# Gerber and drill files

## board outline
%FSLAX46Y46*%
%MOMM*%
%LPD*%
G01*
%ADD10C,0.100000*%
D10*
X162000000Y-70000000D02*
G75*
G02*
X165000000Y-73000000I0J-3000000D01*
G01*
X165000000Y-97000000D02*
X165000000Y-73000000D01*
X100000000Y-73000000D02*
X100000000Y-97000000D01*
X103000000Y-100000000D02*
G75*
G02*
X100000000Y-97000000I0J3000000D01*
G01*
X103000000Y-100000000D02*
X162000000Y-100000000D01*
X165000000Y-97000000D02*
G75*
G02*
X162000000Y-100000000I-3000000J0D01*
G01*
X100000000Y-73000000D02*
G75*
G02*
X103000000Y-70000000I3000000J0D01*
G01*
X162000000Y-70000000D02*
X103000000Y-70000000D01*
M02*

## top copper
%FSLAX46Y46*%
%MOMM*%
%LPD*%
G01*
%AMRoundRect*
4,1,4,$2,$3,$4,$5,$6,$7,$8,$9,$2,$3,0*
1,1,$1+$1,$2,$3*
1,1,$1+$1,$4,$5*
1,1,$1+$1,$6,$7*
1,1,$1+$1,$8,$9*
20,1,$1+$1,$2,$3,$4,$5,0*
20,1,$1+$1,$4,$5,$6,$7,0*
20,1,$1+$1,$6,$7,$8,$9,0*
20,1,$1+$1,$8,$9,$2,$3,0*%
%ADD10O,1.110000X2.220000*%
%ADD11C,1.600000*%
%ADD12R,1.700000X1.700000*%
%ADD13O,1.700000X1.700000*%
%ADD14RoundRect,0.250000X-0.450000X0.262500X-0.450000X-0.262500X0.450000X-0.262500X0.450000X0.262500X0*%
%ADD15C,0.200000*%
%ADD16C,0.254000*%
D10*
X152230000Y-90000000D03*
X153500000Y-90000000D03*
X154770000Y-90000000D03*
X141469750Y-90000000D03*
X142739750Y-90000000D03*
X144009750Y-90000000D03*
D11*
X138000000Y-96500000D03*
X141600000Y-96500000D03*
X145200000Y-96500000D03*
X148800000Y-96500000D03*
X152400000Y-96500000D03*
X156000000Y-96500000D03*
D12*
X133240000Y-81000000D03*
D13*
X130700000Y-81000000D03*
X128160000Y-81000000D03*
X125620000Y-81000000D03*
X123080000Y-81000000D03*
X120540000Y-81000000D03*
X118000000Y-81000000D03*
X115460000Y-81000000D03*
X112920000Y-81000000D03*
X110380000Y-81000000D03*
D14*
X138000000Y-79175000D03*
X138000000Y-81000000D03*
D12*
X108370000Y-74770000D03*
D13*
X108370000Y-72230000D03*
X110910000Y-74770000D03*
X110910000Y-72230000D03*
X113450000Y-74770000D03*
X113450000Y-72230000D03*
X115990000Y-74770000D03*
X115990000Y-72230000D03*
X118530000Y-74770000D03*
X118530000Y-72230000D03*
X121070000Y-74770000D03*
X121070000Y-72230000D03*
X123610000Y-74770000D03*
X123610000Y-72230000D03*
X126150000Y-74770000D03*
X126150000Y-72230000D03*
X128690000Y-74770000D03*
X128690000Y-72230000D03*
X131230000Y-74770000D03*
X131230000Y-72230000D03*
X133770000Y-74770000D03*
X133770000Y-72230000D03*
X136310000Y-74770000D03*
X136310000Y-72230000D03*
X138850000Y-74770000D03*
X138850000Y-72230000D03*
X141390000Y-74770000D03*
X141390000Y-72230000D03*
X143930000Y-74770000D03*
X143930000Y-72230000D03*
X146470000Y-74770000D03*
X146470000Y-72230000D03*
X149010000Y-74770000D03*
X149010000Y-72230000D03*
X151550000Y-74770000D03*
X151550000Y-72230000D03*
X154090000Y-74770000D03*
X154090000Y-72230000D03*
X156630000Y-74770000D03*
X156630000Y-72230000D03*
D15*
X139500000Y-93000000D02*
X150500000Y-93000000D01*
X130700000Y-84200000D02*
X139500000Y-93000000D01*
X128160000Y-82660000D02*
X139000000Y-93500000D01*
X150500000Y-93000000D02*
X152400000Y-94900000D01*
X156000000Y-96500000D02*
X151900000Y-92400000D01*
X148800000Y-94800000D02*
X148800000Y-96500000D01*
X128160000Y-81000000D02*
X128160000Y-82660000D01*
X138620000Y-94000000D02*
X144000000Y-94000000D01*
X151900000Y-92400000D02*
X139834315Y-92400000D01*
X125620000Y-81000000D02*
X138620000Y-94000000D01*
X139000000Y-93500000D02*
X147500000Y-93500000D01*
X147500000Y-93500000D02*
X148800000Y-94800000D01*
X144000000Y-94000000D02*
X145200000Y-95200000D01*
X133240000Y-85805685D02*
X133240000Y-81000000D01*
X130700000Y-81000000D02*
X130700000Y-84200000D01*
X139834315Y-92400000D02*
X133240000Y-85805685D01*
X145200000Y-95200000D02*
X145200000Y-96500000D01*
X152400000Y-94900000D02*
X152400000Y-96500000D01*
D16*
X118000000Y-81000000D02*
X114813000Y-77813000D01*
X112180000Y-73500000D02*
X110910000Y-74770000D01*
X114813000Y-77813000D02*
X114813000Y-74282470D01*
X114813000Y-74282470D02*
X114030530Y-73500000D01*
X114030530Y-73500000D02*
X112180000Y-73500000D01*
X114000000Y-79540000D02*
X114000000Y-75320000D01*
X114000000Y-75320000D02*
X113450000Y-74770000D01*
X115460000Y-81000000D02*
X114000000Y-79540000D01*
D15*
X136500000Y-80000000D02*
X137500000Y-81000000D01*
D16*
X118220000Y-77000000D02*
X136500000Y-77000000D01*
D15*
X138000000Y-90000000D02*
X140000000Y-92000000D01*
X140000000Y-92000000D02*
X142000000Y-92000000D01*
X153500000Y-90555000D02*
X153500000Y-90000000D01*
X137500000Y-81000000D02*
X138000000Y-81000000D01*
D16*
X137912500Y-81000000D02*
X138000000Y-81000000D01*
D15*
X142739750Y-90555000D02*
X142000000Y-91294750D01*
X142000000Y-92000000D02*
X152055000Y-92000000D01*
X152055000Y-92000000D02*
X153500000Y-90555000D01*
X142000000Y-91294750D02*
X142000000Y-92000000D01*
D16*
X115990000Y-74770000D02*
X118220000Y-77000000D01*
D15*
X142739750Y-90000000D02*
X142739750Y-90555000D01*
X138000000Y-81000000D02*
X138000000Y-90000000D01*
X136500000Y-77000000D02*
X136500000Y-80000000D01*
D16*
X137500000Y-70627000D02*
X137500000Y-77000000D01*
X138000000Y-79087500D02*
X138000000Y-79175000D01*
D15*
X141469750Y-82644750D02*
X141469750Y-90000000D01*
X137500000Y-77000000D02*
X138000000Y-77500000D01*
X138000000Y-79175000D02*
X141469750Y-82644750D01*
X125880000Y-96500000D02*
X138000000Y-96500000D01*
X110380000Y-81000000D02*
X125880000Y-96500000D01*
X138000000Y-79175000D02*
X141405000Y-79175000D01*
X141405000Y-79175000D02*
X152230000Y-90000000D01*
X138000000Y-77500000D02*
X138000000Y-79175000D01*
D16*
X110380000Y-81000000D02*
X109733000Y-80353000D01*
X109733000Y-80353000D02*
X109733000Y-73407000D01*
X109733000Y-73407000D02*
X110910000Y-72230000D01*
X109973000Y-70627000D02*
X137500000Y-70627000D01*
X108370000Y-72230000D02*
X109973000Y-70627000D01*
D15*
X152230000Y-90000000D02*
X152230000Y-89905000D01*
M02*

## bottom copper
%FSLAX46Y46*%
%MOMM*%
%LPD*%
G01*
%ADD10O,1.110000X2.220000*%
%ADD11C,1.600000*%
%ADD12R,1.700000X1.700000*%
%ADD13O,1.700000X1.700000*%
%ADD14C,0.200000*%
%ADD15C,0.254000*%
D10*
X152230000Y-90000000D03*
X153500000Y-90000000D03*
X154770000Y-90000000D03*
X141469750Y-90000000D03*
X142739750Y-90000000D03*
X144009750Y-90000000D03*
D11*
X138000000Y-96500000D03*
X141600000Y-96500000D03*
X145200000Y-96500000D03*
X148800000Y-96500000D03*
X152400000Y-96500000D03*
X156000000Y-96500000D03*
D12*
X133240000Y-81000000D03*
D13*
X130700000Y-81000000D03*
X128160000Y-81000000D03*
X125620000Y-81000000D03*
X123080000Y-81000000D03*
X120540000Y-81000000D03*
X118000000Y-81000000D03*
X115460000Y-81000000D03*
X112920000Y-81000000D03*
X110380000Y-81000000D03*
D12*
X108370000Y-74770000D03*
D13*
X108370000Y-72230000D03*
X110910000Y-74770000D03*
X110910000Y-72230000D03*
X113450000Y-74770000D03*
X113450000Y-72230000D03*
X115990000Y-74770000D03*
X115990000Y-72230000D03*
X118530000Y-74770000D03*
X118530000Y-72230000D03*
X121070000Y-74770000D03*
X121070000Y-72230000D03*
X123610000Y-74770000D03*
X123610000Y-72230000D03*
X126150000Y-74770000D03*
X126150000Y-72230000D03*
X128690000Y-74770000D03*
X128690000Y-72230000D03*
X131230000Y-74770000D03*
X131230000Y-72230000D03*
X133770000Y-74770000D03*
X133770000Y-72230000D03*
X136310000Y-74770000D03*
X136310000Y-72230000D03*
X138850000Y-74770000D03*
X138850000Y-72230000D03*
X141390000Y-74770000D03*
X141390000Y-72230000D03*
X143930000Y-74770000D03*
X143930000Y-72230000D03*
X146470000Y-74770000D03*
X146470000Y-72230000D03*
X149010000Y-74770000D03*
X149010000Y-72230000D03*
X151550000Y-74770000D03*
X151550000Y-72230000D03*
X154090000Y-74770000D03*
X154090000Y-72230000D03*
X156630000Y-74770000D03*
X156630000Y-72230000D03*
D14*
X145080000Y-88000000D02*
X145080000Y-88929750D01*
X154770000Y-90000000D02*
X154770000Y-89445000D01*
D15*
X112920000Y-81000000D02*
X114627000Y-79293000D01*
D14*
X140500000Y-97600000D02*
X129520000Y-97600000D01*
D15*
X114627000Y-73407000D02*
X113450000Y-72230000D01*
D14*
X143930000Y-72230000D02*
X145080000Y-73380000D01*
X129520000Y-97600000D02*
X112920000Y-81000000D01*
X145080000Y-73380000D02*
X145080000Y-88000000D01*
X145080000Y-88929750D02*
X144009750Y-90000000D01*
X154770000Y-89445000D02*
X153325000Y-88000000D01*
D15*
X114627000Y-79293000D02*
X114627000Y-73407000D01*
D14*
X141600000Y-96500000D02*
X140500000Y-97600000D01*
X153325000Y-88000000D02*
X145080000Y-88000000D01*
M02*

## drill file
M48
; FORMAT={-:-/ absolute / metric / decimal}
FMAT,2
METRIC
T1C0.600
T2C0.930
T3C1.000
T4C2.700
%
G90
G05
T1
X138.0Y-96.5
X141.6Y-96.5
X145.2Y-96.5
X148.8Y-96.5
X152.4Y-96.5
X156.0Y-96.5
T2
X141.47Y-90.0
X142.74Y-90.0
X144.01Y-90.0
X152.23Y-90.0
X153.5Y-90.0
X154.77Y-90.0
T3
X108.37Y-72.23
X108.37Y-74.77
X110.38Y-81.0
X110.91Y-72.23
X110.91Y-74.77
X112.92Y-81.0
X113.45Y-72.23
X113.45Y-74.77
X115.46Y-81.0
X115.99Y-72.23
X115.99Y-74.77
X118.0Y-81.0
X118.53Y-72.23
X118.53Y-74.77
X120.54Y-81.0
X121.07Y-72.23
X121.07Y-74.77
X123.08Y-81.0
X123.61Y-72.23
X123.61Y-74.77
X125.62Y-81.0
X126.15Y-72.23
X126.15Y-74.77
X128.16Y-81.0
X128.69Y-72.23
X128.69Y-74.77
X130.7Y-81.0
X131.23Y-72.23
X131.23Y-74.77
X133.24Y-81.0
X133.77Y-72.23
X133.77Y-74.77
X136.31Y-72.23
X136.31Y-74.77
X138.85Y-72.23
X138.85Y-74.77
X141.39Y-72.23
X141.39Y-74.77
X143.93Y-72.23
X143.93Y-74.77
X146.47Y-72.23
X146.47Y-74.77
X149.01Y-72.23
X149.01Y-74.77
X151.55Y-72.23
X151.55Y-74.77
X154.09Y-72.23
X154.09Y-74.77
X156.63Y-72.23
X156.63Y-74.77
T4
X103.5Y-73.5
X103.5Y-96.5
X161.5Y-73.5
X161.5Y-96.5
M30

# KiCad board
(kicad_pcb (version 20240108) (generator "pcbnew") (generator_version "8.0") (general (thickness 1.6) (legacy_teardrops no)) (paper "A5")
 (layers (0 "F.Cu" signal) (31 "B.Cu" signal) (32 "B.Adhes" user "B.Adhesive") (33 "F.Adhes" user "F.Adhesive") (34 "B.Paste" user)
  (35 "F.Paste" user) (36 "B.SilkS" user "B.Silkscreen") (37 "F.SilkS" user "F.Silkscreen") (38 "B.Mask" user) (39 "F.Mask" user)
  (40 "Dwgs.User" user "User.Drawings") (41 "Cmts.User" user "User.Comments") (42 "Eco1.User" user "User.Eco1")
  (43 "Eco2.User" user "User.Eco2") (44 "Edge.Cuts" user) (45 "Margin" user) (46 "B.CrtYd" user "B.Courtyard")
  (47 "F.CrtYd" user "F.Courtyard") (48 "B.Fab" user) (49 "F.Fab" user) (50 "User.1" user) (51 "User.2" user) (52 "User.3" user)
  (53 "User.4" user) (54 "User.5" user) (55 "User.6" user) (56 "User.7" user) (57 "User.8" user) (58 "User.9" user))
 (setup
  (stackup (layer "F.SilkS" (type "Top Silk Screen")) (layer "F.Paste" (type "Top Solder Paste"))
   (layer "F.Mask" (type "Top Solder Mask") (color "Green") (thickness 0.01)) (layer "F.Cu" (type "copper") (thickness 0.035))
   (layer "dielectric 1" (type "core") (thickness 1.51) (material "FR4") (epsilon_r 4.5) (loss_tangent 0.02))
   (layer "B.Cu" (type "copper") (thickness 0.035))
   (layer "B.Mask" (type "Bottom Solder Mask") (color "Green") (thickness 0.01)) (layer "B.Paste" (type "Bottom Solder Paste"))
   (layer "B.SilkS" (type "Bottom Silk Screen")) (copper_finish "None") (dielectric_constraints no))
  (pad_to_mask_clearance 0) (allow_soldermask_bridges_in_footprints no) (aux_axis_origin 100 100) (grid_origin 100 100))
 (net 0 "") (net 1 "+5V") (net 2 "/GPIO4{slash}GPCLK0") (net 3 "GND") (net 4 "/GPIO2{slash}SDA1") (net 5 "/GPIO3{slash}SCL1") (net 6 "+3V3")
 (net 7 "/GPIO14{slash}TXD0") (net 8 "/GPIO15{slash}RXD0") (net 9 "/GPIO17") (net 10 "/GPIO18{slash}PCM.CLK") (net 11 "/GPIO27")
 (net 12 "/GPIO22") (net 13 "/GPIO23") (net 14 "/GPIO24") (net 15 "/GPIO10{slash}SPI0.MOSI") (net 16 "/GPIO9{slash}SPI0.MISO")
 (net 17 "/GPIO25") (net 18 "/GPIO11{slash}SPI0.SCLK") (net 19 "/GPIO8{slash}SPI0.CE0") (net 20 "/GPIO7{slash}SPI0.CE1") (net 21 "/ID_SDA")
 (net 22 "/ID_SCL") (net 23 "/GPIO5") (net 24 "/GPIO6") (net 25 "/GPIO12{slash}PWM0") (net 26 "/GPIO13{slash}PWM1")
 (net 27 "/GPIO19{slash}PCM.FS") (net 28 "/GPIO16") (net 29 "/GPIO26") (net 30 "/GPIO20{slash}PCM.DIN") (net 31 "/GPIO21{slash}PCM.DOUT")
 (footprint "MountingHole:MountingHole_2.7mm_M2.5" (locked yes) (layer "F.Cu") (at 161.5 73.5)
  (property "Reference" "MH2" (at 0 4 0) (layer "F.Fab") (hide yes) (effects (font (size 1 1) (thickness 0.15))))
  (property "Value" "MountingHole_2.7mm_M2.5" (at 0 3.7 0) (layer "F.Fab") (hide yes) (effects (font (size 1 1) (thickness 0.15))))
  (pad "" np_thru_hole circle (at 0 0) (size 2.7 2.7) (drill 2.7) (layers "*.Cu" "*.Mask")))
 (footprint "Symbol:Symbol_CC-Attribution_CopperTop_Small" (layer "F.Cu") (at 155.5 79)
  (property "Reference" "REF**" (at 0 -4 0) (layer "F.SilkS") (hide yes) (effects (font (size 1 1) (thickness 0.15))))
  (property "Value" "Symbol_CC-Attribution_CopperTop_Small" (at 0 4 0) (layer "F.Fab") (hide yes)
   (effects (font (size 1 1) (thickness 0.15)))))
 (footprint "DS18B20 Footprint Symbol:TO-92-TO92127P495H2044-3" (layer "F.Cu") (at 153.5 89.23975)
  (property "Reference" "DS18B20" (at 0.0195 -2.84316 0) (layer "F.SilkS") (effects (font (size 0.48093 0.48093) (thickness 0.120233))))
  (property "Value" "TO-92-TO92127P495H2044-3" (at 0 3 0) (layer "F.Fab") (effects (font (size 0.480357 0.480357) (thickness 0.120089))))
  (pad "1" thru_hole oval (at -1.27 0.76025) (size 1.11 2.22) (drill 0.93) (layers "*.Cu" "*.Mask") (remove_unused_layers no) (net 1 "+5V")
   (solder_mask_margin 0.102))
  (pad "2" thru_hole oval (at 0 0.76025) (size 1.11 2.22) (drill 0.93) (layers "*.Cu" "*.Mask") (remove_unused_layers no)
   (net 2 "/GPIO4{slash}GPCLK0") (solder_mask_margin 0.102))
  (pad "3" thru_hole oval (at 1.27 0.76025) (size 1.11 2.22) (drill 0.93) (layers "*.Cu" "*.Mask") (remove_unused_layers no) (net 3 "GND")
   (solder_mask_margin 0.102)))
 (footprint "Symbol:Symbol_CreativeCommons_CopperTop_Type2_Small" (layer "F.Cu") (at 149.5 79)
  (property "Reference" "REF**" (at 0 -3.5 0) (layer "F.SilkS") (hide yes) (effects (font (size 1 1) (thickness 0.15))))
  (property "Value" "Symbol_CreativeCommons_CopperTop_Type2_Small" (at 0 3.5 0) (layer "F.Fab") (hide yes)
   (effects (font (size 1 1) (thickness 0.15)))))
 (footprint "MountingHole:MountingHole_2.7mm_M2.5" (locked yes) (layer "F.Cu") (at 103.5 96.5)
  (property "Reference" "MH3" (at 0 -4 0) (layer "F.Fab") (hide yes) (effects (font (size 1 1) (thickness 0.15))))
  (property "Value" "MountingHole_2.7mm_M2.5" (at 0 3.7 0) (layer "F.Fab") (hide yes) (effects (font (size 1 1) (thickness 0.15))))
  (pad "" np_thru_hole circle (at 0 0) (size 2.7 2.7) (drill 2.7) (layers "*.Cu" "*.Mask")))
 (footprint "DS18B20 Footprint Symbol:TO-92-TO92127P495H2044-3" (layer "F.Cu") (at 142.73975 89.23975)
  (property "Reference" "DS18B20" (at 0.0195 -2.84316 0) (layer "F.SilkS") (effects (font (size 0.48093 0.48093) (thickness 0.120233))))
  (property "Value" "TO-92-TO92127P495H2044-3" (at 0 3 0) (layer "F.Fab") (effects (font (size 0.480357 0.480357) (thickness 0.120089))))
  (pad "1" thru_hole oval (at -1.27 0.76025) (size 1.11 2.22) (drill 0.93) (layers "*.Cu" "*.Mask") (remove_unused_layers no) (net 1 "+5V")
   (solder_mask_margin 0.102))
  (pad "2" thru_hole oval (at 0 0.76025) (size 1.11 2.22) (drill 0.93) (layers "*.Cu" "*.Mask") (remove_unused_layers no)
   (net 2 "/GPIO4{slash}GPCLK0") (solder_mask_margin 0.102))
  (pad "3" thru_hole oval (at 1.27 0.76025) (size 1.11 2.22) (drill 0.93) (layers "*.Cu" "*.Mask") (remove_unused_layers no) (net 3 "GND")
   (solder_mask_margin 0.102)))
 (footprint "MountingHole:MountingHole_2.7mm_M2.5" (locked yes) (layer "F.Cu") (at 103.5 73.5)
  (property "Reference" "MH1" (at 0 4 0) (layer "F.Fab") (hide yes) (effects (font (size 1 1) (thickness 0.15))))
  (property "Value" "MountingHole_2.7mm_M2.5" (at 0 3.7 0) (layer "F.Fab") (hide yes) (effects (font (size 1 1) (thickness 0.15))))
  (pad "" np_thru_hole circle (at 0 0) (size 2.7 2.7) (drill 2.7) (layers "*.Cu" "*.Mask")))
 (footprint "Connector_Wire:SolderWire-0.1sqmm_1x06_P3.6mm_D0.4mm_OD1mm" (layer "F.Cu") (at 138 96.5)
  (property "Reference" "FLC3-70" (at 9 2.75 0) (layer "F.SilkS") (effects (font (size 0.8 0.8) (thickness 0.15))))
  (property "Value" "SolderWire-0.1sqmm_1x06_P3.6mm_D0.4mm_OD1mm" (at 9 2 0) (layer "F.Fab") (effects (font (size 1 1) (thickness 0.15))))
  (pad "1" thru_hole circle (at 0 0) (size 1.6 1.6) (drill 0.6) (layers "*.Cu" "*.Mask") (remove_unused_layers no) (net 1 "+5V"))
  (pad "2" thru_hole circle (at 3.6 0) (size 1.6 1.6) (drill 0.6) (layers "*.Cu" "*.Mask") (remove_unused_layers no) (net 3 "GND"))
  (pad "3" thru_hole circle (at 7.2 0) (size 1.6 1.6) (drill 0.6) (layers "*.Cu" "*.Mask") (remove_unused_layers no))
  (pad "4" thru_hole circle (at 10.8 0) (size 1.6 1.6) (drill 0.6) (layers "*.Cu" "*.Mask") (remove_unused_layers no))
  (pad "5" thru_hole circle (at 14.4 0) (size 1.6 1.6) (drill 0.6) (layers "*.Cu" "*.Mask") (remove_unused_layers no))
  (pad "6" thru_hole circle (at 18 0) (size 1.6 1.6) (drill 0.6) (layers "*.Cu" "*.Mask") (remove_unused_layers no)))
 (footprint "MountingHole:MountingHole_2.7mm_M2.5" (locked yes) (layer "F.Cu") (at 161.5 96.5)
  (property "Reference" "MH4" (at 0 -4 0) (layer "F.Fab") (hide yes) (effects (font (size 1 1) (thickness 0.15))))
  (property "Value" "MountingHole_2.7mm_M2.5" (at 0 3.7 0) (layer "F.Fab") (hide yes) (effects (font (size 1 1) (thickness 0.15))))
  (pad "" np_thru_hole circle (at 0 0) (size 2.7 2.7) (drill 2.7) (layers "*.Cu" "*.Mask")))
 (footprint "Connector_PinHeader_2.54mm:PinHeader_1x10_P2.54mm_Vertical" (layer "F.Cu") (at 133.24 81 -90)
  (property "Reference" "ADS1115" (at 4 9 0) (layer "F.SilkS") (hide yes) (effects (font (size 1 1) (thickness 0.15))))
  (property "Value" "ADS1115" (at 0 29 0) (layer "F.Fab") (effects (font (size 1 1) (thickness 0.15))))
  (pad "1" thru_hole rect (at 0 0 270) (size 1.7 1.7) (drill 1) (layers "*.Cu" "*.Mask") (remove_unused_layers no))
  (pad "2" thru_hole oval (at 0 2.54 270) (size 1.7 1.7) (drill 1) (layers "*.Cu" "*.Mask") (remove_unused_layers no))
  (pad "3" thru_hole oval (at 0 5.08 270) (size 1.7 1.7) (drill 1) (layers "*.Cu" "*.Mask") (remove_unused_layers no))
  (pad "4" thru_hole oval (at 0 7.62 270) (size 1.7 1.7) (drill 1) (layers "*.Cu" "*.Mask") (remove_unused_layers no))
  (pad "5" thru_hole oval (at 0 10.16 270) (size 1.7 1.7) (drill 1) (layers "*.Cu" "*.Mask") (remove_unused_layers no))
  (pad "6" thru_hole oval (at 0 12.7 270) (size 1.7 1.7) (drill 1) (layers "*.Cu" "*.Mask") (remove_unused_layers no))
  (pad "7" thru_hole oval (at 0 15.24 270) (size 1.7 1.7) (drill 1) (layers "*.Cu" "*.Mask") (remove_unused_layers no)
   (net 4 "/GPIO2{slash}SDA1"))
  (pad "8" thru_hole oval (at 0 17.78 270) (size 1.7 1.7) (drill 1) (layers "*.Cu" "*.Mask") (remove_unused_layers no)
   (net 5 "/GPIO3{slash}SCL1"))
  (pad "9" thru_hole oval (at 0 20.32 270) (size 1.7 1.7) (drill 1) (layers "*.Cu" "*.Mask") (remove_unused_layers no) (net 3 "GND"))
  (pad "10" thru_hole oval (at 0 22.86 270) (size 1.7 1.7) (drill 1) (layers "*.Cu" "*.Mask") (remove_unused_layers no) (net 1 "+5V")))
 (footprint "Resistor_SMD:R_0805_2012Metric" (layer "F.Cu") (at 138 80.0875 -90)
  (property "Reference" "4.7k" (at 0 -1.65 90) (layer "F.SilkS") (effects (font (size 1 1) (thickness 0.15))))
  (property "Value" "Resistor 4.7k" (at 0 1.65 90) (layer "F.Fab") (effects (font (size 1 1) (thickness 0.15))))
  (pad "1" smd roundrect (at -0.9125 0 270) (size 1.025 1.4) (layers "F.Cu" "F.Paste" "F.Mask") (roundrect_rratio 0.243902) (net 1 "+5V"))
  (pad "2" smd roundrect (at 0.9125 0 270) (size 1.025 1.4) (layers "F.Cu" "F.Paste" "F.Mask") (roundrect_rratio 0.243902)
   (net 2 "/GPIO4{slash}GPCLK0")))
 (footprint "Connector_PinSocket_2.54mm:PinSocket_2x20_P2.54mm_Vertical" (layer "B.Cu") (at 108.37 74.77 -90)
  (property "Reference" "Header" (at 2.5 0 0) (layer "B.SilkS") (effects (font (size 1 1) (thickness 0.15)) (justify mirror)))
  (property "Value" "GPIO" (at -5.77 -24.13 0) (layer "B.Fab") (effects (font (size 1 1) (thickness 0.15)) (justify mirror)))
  (pad "1" thru_hole rect (at 0 0 270) (size 1.7 1.7) (drill 1) (layers "*.Cu" "*.Mask") (remove_unused_layers no) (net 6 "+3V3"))
  (pad "2" thru_hole oval (at -2.54 0 270) (size 1.7 1.7) (drill 1) (layers "*.Cu" "*.Mask") (remove_unused_layers no) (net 1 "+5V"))
  (pad "3" thru_hole oval (at 0 -2.54 270) (size 1.7 1.7) (drill 1) (layers "*.Cu" "*.Mask") (remove_unused_layers no)
   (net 4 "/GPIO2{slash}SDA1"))
  (pad "4" thru_hole oval (at -2.54 -2.54 270) (size 1.7 1.7) (drill 1) (layers "*.Cu" "*.Mask") (remove_unused_layers no) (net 1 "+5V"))
  (pad "5" thru_hole oval (at 0 -5.08 270) (size 1.7 1.7) (drill 1) (layers "*.Cu" "*.Mask") (remove_unused_layers no)
   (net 5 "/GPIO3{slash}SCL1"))
  (pad "6" thru_hole oval (at -2.54 -5.08 270) (size 1.7 1.7) (drill 1) (layers "*.Cu" "*.Mask") (remove_unused_layers no) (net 3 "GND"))
  (pad "7" thru_hole oval (at 0 -7.62 270) (size 1.7 1.7) (drill 1) (layers "*.Cu" "*.Mask") (remove_unused_layers no)
   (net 2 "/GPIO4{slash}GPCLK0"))
  (pad "8" thru_hole oval (at -2.54 -7.62 270) (size 1.7 1.7) (drill 1) (layers "*.Cu" "*.Mask") (remove_unused_layers no)
   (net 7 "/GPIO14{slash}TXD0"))
  (pad "9" thru_hole oval (at 0 -10.16 270) (size 1.7 1.7) (drill 1) (layers "*.Cu" "*.Mask") (remove_unused_layers no) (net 3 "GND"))
  (pad "10" thru_hole oval (at -2.54 -10.16 270) (size 1.7 1.7) (drill 1) (layers "*.Cu" "*.Mask") (remove_unused_layers no)
   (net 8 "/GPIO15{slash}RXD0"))
  (pad "11" thru_hole oval (at 0 -12.7 270) (size 1.7 1.7) (drill 1) (layers "*.Cu" "*.Mask") (remove_unused_layers no) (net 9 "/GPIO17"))
  (pad "12" thru_hole oval (at -2.54 -12.7 270) (size 1.7 1.7) (drill 1) (layers "*.Cu" "*.Mask") (remove_unused_layers no)
   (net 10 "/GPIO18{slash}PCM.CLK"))
  (pad "13" thru_hole oval (at 0 -15.24 270) (size 1.7 1.7) (drill 1) (layers "*.Cu" "*.Mask") (remove_unused_layers no) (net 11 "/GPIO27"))
  (pad "14" thru_hole oval (at -2.54 -15.24 270) (size 1.7 1.7) (drill 1) (layers "*.Cu" "*.Mask") (remove_unused_layers no) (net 3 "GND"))
  (pad "15" thru_hole oval (at 0 -17.78 270) (size 1.7 1.7) (drill 1) (layers "*.Cu" "*.Mask") (remove_unused_layers no) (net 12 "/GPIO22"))
  (pad "16" thru_hole oval (at -2.54 -17.78 270) (size 1.7 1.7) (drill 1) (layers "*.Cu" "*.Mask") (remove_unused_layers no)
   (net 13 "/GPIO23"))
  (pad "17" thru_hole oval (at 0 -20.32 270) (size 1.7 1.7) (drill 1) (layers "*.Cu" "*.Mask") (remove_unused_layers no) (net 6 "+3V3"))
  (pad "18" thru_hole oval (at -2.54 -20.32 270) (size 1.7 1.7) (drill 1) (layers "*.Cu" "*.Mask") (remove_unused_layers no)
   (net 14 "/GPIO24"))
  (pad "19" thru_hole oval (at 0 -22.86 270) (size 1.7 1.7) (drill 1) (layers "*.Cu" "*.Mask") (remove_unused_layers no)
   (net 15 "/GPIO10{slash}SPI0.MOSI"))
  (pad "20" thru_hole oval (at -2.54 -22.86 270) (size 1.7 1.7) (drill 1) (layers "*.Cu" "*.Mask") (remove_unused_layers no) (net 3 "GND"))
  (pad "21" thru_hole oval (at 0 -25.4 270) (size 1.7 1.7) (drill 1) (layers "*.Cu" "*.Mask") (remove_unused_layers no)
   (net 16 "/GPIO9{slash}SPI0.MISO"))
  (pad "22" thru_hole oval (at -2.54 -25.4 270) (size 1.7 1.7) (drill 1) (layers "*.Cu" "*.Mask") (remove_unused_layers no)
   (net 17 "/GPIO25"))
  (pad "23" thru_hole oval (at 0 -27.94 270) (size 1.7 1.7) (drill 1) (layers "*.Cu" "*.Mask") (remove_unused_layers no)
   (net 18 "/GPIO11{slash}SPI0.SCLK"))
  (pad "24" thru_hole oval (at -2.54 -27.94 270) (size 1.7 1.7) (drill 1) (layers "*.Cu" "*.Mask") (remove_unused_layers no)
   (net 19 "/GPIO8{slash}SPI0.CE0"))
  (pad "25" thru_hole oval (at 0 -30.48 270) (size 1.7 1.7) (drill 1) (layers "*.Cu" "*.Mask") (remove_unused_layers no) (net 3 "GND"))
  (pad "26" thru_hole oval (at -2.54 -30.48 270) (size 1.7 1.7) (drill 1) (layers "*.Cu" "*.Mask") (remove_unused_layers no)
   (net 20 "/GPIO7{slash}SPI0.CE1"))
  (pad "27" thru_hole oval (at 0 -33.02 270) (size 1.7 1.7) (drill 1) (layers "*.Cu" "*.Mask") (remove_unused_layers no) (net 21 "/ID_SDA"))
  (pad "28" thru_hole oval (at -2.54 -33.02 270) (size 1.7 1.7) (drill 1) (layers "*.Cu" "*.Mask") (remove_unused_layers no)
   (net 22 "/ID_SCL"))
  (pad "29" thru_hole oval (at 0 -35.56 270) (size 1.7 1.7) (drill 1) (layers "*.Cu" "*.Mask") (remove_unused_layers no) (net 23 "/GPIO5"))
  (pad "30" thru_hole oval (at -2.54 -35.56 270) (size 1.7 1.7) (drill 1) (layers "*.Cu" "*.Mask") (remove_unused_layers no) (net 3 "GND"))
  (pad "31" thru_hole oval (at 0 -38.1 270) (size 1.7 1.7) (drill 1) (layers "*.Cu" "*.Mask") (remove_unused_layers no) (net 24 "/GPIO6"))
  (pad "32" thru_hole oval (at -2.54 -38.1 270) (size 1.7 1.7) (drill 1) (layers "*.Cu" "*.Mask") (remove_unused_layers no)
   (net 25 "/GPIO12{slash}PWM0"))
  (pad "33" thru_hole oval (at 0 -40.64 270) (size 1.7 1.7) (drill 1) (layers "*.Cu" "*.Mask") (remove_unused_layers no)
   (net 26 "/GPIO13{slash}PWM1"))
  (pad "34" thru_hole oval (at -2.54 -40.64 270) (size 1.7 1.7) (drill 1) (layers "*.Cu" "*.Mask") (remove_unused_layers no) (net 3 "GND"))
  (pad "35" thru_hole oval (at 0 -43.18 270) (size 1.7 1.7) (drill 1) (layers "*.Cu" "*.Mask") (remove_unused_layers no)
   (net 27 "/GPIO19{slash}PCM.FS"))
  (pad "36" thru_hole oval (at -2.54 -43.18 270) (size 1.7 1.7) (drill 1) (layers "*.Cu" "*.Mask") (remove_unused_layers no)
   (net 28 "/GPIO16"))
  (pad "37" thru_hole oval (at 0 -45.72 270) (size 1.7 1.7) (drill 1) (layers "*.Cu" "*.Mask") (remove_unused_layers no) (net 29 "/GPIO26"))
  (pad "38" thru_hole oval (at -2.54 -45.72 270) (size 1.7 1.7) (drill 1) (layers "*.Cu" "*.Mask") (remove_unused_layers no)
   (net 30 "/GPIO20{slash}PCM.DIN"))
  (pad "39" thru_hole oval (at 0 -48.26 270) (size 1.7 1.7) (drill 1) (layers "*.Cu" "*.Mask") (remove_unused_layers no) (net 3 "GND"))
  (pad "40" thru_hole oval (at -2.54 -48.26 270) (size 1.7 1.7) (drill 1) (layers "*.Cu" "*.Mask") (remove_unused_layers no)
   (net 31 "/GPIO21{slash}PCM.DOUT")))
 (gr_arc (start 162 70) (mid 164.12132 70.87868) (end 165 73) (stroke (width 0.1) (type solid)) (layer "Edge.Cuts"))
 (gr_line (start 165 97) (end 165 73) (stroke (width 0.1) (type solid)) (layer "Edge.Cuts"))
 (gr_line (start 100 73) (end 100 97) (stroke (width 0.1) (type solid)) (layer "Edge.Cuts"))
 (gr_arc (start 103 100) (mid 100.87868 99.12132) (end 100 97) (stroke (width 0.1) (type solid)) (layer "Edge.Cuts"))
 (gr_line (start 103 100) (end 162 100) (stroke (width 0.1) (type solid)) (layer "Edge.Cuts"))
 (gr_arc (start 165 97) (mid 164.12132 99.12132) (end 162 100) (stroke (width 0.1) (type solid)) (layer "Edge.Cuts"))
 (gr_arc (start 100 73) (mid 100.87868 70.87868) (end 103 70) (stroke (width 0.1) (type solid)) (layer "Edge.Cuts"))
 (gr_line (start 162 70) (end 103 70) (stroke (width 0.1) (type solid)) (layer "Edge.Cuts"))
 (segment (start 139.5 93) (end 150.5 93) (width 0.2) (layer "F.Cu") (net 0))
 (segment (start 130.7 84.2) (end 139.5 93) (width 0.2) (layer "F.Cu") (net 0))
 (segment (start 128.16 82.66) (end 139 93.5) (width 0.2) (layer "F.Cu") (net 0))
 (segment (start 150.5 93) (end 152.4 94.9) (width 0.2) (layer "F.Cu") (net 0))
 (segment (start 156 96.5) (end 151.9 92.4) (width 0.2) (layer "F.Cu") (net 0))
 (segment (start 148.8 94.8) (end 148.8 96.5) (width 0.2) (layer "F.Cu") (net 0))
 (segment (start 128.16 81) (end 128.16 82.66) (width 0.2) (layer "F.Cu") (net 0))
 (segment (start 138.62 94) (end 144 94) (width 0.2) (layer "F.Cu") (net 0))
 (segment (start 151.9 92.4) (end 139.834315 92.4) (width 0.2) (layer "F.Cu") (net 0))
 (segment (start 125.62 81) (end 138.62 94) (width 0.2) (layer "F.Cu") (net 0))
 (segment (start 139 93.5) (end 147.5 93.5) (width 0.2) (layer "F.Cu") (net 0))
 (segment (start 147.5 93.5) (end 148.8 94.8) (width 0.2) (layer "F.Cu") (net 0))
 (segment (start 144 94) (end 145.2 95.2) (width 0.2) (layer "F.Cu") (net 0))
 (segment (start 133.24 85.805685) (end 133.24 81) (width 0.2) (layer "F.Cu") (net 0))
 (segment (start 130.7 81) (end 130.7 84.2) (width 0.2) (layer "F.Cu") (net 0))
 (segment (start 139.834315 92.4) (end 133.24 85.805685) (width 0.2) (layer "F.Cu") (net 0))
 (segment (start 145.2 95.2) (end 145.2 96.5) (width 0.2) (layer "F.Cu") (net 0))
 (segment (start 152.4 94.9) (end 152.4 96.5) (width 0.2) (layer "F.Cu") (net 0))
 (segment (start 145.08 88) (end 145.08 88.92975) (width 0.2) (layer "B.Cu") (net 3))
 (segment (start 154.77 90) (end 154.77 89.445) (width 0.2) (layer "B.Cu") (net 3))
 (segment (start 112.92 81) (end 114.627 79.293) (width 0.254) (layer "B.Cu") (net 3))
 (segment (start 140.5 97.6) (end 129.52 97.6) (width 0.2) (layer "B.Cu") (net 3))
 (segment (start 114.627 73.407) (end 113.45 72.23) (width 0.254) (layer "B.Cu") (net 3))
 (segment (start 143.93 72.23) (end 145.08 73.38) (width 0.2) (layer "B.Cu") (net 3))
 (segment (start 129.52 97.6) (end 112.92 81) (width 0.2) (layer "B.Cu") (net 3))
 (segment (start 145.08 73.38) (end 145.08 88) (width 0.2) (layer "B.Cu") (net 3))
 (segment (start 145.08 88.92975) (end 144.00975 90) (width 0.2) (layer "B.Cu") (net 3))
 (segment (start 154.77 89.445) (end 153.325 88) (width 0.2) (layer "B.Cu") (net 3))
 (segment (start 114.627 79.293) (end 114.627 73.407) (width 0.254) (layer "B.Cu") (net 3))
 (segment (start 141.6 96.5) (end 140.5 97.6) (width 0.2) (layer "B.Cu") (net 3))
 (segment (start 153.325 88) (end 145.08 88) (width 0.2) (layer "B.Cu") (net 3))
 (segment (start 118 81) (end 114.813 77.813) (width 0.254) (layer "F.Cu") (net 4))
 (segment (start 112.18 73.5) (end 110.91 74.77) (width 0.254) (layer "F.Cu") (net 4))
 (segment (start 114.813 77.813) (end 114.813 74.28247) (width 0.254) (layer "F.Cu") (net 4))
 (segment (start 114.813 74.28247) (end 114.03053 73.5) (width 0.254) (layer "F.Cu") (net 4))
 (segment (start 114.03053 73.5) (end 112.18 73.5) (width 0.254) (layer "F.Cu") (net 4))
 (segment (start 114 79.54) (end 114 75.32) (width 0.254) (layer "F.Cu") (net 5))
 (segment (start 114 75.32) (end 113.45 74.77) (width 0.254) (layer "F.Cu") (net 5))
 (segment (start 115.46 81) (end 114 79.54) (width 0.254) (layer "F.Cu") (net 5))
 (segment (start 136.5 80) (end 137.5 81) (width 0.2) (layer "F.Cu") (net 2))
 (segment (start 118.22 77) (end 136.5 77) (width 0.254) (layer "F.Cu") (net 2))
 (segment (start 138 90) (end 140 92) (width 0.2) (layer "F.Cu") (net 2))
 (segment (start 140 92) (end 142 92) (width 0.2) (layer "F.Cu") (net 2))
 (segment (start 153.5 90.555) (end 153.5 90) (width 0.2) (layer "F.Cu") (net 2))
 (segment (start 137.5 81) (end 138 81) (width 0.2) (layer "F.Cu") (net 2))
 (segment (start 137.9125 81) (end 138 81) (width 0.254) (layer "F.Cu") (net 2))
 (segment (start 142.73975 90.555) (end 142 91.29475) (width 0.2) (layer "F.Cu") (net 2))
 (segment (start 142 92) (end 152.055 92) (width 0.2) (layer "F.Cu") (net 2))
 (segment (start 152.055 92) (end 153.5 90.555) (width 0.2) (layer "F.Cu") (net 2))
 (segment (start 142 91.29475) (end 142 92) (width 0.2) (layer "F.Cu") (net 2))
 (segment (start 115.99 74.77) (end 118.22 77) (width 0.254) (layer "F.Cu") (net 2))
 (segment (start 142.73975 90) (end 142.73975 90.555) (width 0.2) (layer "F.Cu") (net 2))
 (segment (start 138 81) (end 138 90) (width 0.2) (layer "F.Cu") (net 2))
 (segment (start 136.5 77) (end 136.5 80) (width 0.2) (layer "F.Cu") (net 2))
 (segment (start 137.5 70.627) (end 137.5 77) (width 0.254) (layer "F.Cu") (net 1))
 (segment (start 138 79.0875) (end 138 79.175) (width 0.254) (layer "F.Cu") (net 1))
 (segment (start 141.46975 82.64475) (end 141.46975 90) (width 0.2) (layer "F.Cu") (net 1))
 (segment (start 137.5 77) (end 138 77.5) (width 0.2) (layer "F.Cu") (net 1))
 (segment (start 138 79.175) (end 141.46975 82.64475) (width 0.2) (layer "F.Cu") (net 1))
 (segment (start 125.88 96.5) (end 138 96.5) (width 0.2) (layer "F.Cu") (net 1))
 (segment (start 110.38 81) (end 125.88 96.5) (width 0.2) (layer "F.Cu") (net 1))
 (segment (start 138 79.175) (end 141.405 79.175) (width 0.2) (layer "F.Cu") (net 1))
 (segment (start 141.405 79.175) (end 152.23 90) (width 0.2) (layer "F.Cu") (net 1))
 (segment (start 138 77.5) (end 138 79.175) (width 0.2) (layer "F.Cu") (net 1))
 (segment (start 110.38 81) (end 109.733 80.353) (width 0.254) (layer "F.Cu") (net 1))
 (segment (start 109.733 80.353) (end 109.733 73.407) (width 0.254) (layer "F.Cu") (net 1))
 (segment (start 109.733 73.407) (end 110.91 72.23) (width 0.254) (layer "F.Cu") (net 1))
 (segment (start 109.973 70.627) (end 137.5 70.627) (width 0.254) (layer "F.Cu") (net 1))
 (segment (start 108.37 72.23) (end 109.973 70.627) (width 0.254) (layer "F.Cu") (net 1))
 (segment (start 152.23 90) (end 152.23 89.905) (width 0.2) (layer "F.Cu") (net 1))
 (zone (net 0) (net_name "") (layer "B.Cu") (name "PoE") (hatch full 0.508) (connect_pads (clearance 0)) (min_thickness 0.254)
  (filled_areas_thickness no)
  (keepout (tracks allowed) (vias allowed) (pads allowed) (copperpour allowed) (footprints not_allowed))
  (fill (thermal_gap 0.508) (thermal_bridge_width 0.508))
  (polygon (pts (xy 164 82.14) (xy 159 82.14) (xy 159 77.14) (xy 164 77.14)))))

